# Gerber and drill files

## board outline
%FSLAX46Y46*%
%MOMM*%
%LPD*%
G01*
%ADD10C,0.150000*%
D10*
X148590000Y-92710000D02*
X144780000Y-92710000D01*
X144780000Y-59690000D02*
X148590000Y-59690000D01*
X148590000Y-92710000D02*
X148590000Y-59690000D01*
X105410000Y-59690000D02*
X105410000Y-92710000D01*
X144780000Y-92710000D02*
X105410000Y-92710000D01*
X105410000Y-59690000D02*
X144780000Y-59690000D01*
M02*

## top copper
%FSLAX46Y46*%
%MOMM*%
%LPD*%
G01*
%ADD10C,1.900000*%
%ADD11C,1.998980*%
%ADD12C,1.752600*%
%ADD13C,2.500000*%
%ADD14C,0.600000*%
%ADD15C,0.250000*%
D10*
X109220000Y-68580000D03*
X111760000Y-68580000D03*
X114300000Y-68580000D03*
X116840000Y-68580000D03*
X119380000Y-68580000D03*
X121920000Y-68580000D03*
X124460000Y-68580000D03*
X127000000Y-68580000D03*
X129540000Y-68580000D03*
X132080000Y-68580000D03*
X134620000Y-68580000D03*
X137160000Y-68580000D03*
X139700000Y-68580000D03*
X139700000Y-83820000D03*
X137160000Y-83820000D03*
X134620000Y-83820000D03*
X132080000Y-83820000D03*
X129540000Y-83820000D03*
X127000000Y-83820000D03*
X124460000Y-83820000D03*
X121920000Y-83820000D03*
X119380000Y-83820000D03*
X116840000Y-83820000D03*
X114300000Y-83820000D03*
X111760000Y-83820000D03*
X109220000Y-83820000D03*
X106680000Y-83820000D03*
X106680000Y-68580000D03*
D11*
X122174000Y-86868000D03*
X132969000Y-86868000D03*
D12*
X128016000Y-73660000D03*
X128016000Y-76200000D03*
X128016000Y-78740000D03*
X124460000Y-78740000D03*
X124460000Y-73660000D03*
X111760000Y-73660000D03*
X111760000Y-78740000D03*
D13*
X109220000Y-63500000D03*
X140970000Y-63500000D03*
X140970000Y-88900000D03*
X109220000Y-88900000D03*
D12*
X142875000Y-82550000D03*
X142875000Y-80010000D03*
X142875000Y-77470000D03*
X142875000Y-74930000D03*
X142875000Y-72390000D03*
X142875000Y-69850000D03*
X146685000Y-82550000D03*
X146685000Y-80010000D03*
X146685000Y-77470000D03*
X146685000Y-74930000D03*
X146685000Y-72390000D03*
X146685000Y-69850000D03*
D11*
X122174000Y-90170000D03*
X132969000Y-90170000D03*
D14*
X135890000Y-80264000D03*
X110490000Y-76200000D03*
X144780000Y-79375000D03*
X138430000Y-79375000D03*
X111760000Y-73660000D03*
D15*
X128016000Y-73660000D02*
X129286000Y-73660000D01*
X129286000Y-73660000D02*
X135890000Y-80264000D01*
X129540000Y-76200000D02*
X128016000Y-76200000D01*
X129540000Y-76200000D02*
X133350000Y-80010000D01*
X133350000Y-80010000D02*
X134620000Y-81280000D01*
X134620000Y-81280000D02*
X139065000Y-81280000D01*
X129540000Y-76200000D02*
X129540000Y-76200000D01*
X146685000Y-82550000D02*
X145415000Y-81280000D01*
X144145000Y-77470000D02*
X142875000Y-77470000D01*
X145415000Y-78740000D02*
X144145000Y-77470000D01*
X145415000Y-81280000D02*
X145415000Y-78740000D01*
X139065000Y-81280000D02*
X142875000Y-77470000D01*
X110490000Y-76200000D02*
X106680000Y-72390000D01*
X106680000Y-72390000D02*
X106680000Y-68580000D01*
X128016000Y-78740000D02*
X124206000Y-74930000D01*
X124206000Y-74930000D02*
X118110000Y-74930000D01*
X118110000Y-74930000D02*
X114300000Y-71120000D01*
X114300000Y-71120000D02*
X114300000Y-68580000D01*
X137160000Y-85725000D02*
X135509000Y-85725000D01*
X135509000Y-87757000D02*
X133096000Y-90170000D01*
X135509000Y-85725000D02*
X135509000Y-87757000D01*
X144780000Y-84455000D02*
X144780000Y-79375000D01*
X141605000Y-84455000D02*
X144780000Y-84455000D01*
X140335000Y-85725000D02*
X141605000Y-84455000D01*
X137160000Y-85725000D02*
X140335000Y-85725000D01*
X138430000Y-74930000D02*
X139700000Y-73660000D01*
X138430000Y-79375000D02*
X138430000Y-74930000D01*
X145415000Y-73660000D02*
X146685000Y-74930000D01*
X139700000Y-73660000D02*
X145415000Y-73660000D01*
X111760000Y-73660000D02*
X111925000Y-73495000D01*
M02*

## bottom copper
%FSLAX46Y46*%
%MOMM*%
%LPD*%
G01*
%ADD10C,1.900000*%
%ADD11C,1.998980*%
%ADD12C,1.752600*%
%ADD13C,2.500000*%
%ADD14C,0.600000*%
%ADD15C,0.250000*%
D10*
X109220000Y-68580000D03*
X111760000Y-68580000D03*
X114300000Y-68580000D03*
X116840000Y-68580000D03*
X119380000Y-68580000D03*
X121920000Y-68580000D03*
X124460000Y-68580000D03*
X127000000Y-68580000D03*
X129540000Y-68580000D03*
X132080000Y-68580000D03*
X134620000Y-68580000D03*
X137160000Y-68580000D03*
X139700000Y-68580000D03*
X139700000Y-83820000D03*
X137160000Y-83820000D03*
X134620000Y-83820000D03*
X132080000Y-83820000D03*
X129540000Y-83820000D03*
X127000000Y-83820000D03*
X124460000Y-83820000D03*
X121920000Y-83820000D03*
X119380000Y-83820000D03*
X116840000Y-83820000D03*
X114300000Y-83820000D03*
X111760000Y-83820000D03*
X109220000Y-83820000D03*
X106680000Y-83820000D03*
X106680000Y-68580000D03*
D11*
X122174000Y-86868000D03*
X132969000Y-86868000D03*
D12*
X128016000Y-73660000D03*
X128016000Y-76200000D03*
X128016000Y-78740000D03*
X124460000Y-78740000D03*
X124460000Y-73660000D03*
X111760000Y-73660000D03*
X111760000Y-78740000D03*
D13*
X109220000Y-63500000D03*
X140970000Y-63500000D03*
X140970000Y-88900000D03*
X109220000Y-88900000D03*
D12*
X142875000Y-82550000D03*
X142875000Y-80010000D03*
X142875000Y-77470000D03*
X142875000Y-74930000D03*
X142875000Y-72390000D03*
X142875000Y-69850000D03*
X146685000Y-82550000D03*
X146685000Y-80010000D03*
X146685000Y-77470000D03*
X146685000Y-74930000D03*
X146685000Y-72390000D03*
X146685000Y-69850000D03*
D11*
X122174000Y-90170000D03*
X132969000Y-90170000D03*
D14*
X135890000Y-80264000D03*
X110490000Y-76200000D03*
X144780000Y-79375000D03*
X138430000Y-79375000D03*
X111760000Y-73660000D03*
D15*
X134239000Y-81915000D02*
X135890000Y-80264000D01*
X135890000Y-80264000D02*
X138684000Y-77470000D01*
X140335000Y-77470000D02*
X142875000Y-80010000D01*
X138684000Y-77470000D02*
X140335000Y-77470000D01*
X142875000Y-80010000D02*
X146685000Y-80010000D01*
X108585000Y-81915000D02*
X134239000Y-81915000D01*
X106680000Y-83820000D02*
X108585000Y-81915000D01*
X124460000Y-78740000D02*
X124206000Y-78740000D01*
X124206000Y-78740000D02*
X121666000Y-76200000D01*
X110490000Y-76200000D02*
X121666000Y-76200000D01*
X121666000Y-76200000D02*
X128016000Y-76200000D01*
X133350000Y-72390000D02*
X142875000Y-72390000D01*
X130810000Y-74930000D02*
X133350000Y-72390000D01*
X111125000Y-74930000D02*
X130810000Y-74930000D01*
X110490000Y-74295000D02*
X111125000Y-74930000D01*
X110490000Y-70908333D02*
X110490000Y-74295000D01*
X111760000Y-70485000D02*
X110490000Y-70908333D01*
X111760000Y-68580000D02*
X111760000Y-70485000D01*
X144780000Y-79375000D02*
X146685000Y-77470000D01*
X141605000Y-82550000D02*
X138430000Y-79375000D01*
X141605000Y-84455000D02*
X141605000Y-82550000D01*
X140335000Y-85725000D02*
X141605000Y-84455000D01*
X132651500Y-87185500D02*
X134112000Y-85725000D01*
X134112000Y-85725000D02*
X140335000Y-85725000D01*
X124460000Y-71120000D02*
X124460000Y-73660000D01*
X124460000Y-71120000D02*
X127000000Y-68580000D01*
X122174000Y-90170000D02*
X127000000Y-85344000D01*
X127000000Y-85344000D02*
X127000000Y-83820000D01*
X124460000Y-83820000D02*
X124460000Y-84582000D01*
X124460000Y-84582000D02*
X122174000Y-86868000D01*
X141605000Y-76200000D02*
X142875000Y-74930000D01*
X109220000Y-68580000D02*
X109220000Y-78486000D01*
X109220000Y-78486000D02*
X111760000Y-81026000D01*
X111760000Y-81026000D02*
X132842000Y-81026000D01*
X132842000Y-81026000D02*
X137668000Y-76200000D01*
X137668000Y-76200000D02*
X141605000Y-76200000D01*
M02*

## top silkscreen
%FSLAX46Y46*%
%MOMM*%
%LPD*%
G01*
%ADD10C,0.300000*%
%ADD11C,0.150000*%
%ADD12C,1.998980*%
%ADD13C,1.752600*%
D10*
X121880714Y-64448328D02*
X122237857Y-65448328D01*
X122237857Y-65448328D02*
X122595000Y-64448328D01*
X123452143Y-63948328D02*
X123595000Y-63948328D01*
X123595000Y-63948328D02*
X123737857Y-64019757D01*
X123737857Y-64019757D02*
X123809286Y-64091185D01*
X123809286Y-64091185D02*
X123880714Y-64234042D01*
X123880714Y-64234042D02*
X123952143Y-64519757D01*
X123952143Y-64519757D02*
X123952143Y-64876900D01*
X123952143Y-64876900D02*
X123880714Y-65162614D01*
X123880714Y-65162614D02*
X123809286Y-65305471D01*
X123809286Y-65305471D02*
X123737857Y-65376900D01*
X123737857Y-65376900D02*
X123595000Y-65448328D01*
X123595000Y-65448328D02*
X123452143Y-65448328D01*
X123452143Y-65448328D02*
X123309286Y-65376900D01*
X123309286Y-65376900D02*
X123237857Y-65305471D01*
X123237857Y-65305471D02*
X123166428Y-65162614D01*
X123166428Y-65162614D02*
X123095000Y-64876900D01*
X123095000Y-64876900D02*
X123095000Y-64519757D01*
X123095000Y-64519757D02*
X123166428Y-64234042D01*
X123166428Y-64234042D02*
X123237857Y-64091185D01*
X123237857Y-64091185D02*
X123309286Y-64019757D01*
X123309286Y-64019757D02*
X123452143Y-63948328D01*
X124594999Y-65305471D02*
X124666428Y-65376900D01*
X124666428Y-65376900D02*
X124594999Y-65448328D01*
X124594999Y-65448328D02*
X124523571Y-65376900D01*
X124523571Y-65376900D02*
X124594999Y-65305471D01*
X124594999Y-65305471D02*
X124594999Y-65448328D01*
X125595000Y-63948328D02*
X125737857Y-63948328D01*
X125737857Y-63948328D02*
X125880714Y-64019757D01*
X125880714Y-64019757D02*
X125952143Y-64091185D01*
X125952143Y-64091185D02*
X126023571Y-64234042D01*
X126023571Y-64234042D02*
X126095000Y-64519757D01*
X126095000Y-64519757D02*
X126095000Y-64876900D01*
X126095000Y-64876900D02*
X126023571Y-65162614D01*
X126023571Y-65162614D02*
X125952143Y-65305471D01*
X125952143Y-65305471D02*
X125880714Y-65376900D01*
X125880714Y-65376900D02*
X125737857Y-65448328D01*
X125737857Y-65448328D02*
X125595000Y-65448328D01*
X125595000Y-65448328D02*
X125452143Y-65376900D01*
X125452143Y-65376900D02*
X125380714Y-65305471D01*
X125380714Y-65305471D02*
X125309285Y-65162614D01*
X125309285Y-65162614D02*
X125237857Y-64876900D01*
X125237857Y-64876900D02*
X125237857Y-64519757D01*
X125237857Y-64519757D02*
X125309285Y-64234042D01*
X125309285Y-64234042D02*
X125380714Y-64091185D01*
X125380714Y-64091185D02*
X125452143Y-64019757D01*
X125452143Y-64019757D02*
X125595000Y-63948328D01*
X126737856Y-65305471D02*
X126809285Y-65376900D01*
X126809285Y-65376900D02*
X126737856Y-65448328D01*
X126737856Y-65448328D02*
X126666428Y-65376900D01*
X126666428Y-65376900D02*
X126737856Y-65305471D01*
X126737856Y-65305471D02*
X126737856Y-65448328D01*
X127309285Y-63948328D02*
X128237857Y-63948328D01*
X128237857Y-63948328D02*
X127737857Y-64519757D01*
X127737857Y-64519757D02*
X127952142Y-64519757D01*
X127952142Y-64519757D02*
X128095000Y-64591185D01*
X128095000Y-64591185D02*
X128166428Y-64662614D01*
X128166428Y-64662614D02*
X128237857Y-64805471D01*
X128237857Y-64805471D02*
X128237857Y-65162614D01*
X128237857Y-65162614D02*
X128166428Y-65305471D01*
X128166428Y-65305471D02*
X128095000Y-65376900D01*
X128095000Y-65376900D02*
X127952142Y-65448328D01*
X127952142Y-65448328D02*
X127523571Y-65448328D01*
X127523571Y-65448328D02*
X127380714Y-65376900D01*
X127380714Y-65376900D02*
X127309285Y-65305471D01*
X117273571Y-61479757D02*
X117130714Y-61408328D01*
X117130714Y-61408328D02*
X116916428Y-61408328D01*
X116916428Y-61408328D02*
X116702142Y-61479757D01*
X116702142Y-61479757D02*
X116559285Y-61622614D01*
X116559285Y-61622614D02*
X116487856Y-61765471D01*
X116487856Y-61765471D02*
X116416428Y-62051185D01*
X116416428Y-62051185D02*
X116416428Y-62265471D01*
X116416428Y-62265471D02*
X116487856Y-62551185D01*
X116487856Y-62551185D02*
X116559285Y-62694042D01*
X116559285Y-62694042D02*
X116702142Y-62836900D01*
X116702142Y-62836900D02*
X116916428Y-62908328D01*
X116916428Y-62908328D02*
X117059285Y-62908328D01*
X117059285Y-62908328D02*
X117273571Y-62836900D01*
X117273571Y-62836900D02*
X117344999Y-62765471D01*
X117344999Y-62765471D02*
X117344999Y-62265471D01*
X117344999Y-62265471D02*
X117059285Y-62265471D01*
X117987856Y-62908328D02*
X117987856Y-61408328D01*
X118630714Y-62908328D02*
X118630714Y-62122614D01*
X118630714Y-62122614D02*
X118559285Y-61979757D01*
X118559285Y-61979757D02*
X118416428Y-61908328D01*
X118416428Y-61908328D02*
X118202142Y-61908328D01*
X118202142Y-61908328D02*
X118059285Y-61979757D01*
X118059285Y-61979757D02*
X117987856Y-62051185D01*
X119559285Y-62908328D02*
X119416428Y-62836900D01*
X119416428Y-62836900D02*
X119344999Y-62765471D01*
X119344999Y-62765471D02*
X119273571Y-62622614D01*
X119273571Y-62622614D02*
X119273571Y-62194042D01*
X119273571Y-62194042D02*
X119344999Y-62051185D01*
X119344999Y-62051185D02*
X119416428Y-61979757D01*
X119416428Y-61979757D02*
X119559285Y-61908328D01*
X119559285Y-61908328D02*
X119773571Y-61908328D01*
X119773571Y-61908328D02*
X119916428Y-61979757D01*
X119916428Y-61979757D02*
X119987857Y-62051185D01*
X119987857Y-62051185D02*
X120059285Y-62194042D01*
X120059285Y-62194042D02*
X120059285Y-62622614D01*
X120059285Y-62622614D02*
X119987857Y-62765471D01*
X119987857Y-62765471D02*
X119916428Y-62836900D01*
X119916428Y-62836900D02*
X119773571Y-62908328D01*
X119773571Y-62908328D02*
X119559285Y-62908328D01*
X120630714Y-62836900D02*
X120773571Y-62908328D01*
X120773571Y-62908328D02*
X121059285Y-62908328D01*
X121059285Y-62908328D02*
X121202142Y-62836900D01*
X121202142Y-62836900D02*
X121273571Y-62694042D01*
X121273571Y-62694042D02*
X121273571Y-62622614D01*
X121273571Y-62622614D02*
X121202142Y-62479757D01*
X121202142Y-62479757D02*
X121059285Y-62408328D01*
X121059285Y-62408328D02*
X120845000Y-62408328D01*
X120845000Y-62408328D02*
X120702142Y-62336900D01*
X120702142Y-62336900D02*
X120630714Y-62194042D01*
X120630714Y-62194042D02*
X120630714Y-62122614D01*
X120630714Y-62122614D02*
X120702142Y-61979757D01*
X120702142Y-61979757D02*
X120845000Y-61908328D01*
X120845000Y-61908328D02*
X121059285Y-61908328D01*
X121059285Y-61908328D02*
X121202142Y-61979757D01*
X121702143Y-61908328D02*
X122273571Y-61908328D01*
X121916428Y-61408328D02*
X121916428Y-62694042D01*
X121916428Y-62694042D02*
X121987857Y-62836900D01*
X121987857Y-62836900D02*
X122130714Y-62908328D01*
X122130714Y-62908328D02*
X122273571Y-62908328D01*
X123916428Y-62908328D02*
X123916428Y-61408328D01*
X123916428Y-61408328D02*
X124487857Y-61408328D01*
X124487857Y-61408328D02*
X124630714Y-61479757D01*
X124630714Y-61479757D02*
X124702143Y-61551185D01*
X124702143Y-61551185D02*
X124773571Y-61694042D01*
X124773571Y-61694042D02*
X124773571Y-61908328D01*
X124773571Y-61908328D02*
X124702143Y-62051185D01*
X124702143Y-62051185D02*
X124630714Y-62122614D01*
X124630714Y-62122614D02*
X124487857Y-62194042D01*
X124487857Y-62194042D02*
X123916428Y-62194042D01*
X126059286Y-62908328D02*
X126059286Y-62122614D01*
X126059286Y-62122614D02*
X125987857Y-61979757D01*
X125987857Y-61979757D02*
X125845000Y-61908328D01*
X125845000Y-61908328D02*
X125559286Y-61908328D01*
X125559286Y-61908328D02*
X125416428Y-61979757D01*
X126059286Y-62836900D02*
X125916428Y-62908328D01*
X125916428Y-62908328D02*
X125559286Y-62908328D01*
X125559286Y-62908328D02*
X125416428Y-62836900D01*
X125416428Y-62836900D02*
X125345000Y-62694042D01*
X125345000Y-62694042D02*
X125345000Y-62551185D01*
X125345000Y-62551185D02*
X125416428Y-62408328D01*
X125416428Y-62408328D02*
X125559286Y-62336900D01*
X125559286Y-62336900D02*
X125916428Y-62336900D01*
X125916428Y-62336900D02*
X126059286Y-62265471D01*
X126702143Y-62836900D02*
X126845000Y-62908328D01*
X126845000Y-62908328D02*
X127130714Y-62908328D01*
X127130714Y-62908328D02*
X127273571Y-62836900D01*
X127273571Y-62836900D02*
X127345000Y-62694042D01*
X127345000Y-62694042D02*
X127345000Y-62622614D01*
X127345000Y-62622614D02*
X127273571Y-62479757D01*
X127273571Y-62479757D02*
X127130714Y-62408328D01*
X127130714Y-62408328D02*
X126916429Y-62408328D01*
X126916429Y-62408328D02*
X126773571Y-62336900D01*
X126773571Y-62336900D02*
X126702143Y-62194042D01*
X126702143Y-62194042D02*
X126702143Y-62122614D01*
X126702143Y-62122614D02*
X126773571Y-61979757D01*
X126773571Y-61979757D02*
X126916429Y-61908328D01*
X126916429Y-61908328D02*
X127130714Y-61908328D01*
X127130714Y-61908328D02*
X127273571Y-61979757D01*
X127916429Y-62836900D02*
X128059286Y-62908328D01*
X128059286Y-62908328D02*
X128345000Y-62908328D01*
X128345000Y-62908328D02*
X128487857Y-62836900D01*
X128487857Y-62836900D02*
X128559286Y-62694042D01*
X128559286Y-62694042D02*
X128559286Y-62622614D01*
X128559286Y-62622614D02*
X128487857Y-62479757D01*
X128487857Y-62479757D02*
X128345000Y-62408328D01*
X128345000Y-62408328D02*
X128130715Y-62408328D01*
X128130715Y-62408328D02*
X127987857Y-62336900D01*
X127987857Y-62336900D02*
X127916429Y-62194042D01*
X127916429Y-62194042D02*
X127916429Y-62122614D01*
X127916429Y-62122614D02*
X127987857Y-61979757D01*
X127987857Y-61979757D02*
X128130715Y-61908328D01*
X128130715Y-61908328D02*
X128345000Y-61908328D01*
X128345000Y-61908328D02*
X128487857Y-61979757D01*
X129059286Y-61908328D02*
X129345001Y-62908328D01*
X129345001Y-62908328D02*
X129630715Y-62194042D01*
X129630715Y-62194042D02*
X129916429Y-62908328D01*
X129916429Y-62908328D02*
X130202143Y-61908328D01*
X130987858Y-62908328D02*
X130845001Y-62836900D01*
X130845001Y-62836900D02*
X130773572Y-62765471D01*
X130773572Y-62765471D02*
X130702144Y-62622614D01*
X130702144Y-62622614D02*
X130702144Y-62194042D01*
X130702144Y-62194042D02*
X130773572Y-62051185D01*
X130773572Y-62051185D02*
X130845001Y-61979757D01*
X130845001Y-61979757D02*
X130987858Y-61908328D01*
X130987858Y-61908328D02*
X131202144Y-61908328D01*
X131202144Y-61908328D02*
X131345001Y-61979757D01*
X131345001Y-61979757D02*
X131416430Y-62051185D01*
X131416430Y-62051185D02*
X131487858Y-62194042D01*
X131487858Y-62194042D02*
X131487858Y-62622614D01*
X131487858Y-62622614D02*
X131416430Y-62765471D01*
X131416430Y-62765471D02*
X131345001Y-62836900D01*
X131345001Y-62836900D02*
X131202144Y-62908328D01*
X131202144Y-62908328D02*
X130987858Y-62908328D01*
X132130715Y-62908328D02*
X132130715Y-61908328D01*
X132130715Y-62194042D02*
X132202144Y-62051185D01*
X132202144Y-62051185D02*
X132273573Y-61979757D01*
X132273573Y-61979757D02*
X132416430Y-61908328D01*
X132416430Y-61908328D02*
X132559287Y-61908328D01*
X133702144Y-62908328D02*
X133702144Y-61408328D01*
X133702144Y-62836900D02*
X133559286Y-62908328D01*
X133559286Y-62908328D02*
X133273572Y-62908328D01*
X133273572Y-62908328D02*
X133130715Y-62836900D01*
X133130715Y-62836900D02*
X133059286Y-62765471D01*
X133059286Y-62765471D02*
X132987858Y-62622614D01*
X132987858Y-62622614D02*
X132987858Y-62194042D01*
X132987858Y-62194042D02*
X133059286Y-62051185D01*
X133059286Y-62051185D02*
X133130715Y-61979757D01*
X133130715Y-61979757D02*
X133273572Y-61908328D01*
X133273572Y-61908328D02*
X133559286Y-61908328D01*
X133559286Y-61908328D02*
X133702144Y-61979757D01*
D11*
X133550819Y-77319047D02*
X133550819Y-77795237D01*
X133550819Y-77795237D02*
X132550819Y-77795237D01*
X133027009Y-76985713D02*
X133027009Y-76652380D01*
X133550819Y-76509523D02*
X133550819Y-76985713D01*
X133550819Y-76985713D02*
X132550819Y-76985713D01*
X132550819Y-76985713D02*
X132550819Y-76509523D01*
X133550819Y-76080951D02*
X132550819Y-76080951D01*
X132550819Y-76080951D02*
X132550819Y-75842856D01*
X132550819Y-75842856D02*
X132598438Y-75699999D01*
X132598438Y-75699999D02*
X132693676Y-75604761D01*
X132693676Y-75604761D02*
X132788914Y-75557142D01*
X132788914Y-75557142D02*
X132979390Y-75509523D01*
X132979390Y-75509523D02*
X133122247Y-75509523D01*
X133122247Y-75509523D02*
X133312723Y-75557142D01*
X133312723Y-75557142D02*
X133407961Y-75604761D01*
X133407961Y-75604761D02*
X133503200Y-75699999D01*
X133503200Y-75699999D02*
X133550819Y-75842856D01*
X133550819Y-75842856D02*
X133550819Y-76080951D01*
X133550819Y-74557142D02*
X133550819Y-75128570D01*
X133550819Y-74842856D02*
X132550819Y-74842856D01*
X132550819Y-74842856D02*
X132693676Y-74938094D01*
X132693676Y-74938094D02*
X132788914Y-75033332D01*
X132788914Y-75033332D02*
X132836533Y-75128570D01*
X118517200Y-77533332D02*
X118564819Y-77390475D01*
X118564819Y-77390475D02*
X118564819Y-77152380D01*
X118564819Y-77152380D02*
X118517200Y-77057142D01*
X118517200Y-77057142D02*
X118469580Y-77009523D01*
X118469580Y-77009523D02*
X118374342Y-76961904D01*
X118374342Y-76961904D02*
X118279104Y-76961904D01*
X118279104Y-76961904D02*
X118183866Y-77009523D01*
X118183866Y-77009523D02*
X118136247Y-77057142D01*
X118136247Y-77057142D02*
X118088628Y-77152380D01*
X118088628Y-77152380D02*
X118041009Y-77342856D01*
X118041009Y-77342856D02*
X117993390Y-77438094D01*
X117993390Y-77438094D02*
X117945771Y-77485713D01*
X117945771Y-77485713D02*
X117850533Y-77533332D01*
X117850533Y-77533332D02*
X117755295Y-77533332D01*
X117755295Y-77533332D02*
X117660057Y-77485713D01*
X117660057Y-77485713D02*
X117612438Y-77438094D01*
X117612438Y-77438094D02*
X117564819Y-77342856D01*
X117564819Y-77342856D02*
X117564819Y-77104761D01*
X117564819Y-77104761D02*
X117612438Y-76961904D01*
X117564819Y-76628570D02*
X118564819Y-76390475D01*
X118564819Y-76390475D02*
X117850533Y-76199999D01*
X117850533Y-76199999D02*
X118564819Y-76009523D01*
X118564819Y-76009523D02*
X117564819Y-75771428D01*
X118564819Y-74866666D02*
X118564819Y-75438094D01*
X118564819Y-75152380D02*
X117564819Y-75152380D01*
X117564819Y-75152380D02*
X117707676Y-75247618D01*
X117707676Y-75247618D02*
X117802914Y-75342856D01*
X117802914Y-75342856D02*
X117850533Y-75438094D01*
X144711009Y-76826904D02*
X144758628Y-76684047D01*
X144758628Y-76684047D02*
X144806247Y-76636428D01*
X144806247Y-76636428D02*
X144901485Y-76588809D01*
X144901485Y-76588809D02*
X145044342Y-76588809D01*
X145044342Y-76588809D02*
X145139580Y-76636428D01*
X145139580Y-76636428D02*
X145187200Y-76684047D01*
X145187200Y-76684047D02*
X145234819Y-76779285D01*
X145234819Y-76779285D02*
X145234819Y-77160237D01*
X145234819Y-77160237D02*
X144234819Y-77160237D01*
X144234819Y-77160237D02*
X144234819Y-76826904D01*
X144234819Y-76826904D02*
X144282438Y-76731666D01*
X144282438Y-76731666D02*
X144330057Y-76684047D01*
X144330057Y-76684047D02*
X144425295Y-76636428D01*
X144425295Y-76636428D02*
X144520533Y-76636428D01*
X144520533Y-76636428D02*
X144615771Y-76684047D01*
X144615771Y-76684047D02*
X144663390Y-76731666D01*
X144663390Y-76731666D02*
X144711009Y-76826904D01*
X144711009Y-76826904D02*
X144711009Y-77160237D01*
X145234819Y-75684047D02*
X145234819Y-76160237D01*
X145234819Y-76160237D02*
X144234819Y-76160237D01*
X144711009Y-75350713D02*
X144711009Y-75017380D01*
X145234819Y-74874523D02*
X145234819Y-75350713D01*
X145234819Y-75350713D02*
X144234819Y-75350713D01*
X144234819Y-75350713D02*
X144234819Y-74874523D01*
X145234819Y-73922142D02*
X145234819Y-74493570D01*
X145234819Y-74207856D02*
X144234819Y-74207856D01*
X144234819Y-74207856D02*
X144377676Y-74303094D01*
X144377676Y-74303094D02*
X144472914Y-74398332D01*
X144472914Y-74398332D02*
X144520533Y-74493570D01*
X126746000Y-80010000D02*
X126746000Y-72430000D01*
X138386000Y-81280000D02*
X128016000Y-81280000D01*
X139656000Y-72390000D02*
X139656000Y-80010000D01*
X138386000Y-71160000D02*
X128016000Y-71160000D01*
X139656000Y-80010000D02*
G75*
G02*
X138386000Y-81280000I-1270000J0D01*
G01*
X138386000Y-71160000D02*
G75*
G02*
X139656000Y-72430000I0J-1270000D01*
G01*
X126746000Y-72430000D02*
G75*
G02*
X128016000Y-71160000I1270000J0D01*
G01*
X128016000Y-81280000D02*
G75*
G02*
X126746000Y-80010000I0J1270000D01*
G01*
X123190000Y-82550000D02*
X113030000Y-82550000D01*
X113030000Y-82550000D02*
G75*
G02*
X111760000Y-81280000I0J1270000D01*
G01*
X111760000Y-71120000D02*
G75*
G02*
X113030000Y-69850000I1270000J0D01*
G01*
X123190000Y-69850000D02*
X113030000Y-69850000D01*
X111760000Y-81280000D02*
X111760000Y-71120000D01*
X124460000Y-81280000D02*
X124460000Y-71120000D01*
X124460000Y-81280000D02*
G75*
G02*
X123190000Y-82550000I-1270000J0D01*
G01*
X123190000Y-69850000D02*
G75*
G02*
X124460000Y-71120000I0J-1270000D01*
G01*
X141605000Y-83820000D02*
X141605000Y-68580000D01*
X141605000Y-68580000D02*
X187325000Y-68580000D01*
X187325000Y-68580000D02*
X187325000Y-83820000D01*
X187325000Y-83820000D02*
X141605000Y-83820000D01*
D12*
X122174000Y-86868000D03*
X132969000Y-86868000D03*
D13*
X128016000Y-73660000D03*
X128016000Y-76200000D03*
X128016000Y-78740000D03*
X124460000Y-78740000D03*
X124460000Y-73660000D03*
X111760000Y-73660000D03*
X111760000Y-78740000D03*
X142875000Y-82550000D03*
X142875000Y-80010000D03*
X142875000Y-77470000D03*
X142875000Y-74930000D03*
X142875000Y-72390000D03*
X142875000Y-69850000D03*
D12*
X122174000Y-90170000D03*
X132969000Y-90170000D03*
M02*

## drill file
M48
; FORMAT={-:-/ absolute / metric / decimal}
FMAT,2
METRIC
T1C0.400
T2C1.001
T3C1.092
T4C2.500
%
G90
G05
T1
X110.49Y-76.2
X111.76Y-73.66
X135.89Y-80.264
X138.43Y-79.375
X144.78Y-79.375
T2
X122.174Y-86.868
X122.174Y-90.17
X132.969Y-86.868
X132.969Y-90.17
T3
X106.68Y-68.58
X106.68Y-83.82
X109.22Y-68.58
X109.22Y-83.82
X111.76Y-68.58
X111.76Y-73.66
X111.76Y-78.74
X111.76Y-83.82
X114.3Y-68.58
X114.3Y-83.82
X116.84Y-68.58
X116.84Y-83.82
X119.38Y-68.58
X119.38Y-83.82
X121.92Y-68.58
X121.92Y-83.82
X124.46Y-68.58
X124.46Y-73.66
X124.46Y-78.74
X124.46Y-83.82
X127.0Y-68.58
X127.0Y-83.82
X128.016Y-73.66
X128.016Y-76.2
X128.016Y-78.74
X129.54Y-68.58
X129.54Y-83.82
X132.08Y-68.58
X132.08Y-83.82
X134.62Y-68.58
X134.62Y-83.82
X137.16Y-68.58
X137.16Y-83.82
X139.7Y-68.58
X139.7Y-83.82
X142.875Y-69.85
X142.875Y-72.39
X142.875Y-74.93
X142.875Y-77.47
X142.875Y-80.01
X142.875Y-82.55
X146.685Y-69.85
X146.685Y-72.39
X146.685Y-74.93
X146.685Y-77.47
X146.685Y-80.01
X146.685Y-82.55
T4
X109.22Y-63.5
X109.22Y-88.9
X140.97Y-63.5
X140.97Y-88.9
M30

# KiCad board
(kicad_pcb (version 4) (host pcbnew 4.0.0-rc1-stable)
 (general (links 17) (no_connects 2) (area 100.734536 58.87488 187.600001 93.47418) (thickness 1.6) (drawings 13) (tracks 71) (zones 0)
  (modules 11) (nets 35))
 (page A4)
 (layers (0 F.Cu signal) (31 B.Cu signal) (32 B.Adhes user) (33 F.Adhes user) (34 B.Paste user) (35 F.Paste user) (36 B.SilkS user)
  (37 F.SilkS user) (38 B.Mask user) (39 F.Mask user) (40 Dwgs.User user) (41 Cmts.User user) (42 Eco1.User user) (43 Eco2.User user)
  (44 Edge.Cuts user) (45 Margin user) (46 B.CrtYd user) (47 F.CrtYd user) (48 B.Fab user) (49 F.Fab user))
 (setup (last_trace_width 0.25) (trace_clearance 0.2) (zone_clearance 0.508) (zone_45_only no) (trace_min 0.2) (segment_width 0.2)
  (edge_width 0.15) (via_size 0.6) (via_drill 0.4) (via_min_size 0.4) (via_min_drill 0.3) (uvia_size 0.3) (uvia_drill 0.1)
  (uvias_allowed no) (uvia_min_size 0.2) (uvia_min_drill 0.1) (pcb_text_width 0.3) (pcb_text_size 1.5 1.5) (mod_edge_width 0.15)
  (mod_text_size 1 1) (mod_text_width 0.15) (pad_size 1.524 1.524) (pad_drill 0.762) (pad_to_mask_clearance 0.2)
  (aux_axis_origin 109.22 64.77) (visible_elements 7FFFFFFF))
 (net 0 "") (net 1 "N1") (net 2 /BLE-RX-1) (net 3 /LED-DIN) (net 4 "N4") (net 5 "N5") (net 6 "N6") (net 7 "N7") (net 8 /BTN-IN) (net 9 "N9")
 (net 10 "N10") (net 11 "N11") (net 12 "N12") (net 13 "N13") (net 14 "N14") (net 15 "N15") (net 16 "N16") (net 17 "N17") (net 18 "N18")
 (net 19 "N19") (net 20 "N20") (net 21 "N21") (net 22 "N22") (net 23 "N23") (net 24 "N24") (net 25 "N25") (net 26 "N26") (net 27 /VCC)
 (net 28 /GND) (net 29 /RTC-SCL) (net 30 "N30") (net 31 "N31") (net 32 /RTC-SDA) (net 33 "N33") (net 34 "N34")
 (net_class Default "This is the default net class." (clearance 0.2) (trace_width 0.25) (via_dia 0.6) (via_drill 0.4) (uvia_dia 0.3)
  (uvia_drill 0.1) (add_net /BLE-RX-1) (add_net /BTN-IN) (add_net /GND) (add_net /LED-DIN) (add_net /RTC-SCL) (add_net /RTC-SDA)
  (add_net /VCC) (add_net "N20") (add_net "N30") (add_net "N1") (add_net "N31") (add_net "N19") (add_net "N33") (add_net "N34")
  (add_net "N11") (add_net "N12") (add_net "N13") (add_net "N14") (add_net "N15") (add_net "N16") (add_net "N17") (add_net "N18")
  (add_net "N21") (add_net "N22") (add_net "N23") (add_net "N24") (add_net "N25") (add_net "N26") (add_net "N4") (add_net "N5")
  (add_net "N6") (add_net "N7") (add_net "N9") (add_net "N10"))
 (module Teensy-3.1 (layer B.Cu) (at 109.22 68.58)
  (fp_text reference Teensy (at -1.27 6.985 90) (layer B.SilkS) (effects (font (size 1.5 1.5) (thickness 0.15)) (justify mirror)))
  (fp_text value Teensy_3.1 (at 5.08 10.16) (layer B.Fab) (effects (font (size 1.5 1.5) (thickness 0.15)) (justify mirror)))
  (pad 0 thru_hole circle (at 0 0) (size 1.9 1.9) (drill 1.0922) (layers *.Cu *.Mask B.SilkS) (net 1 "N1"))
  (pad 1 thru_hole circle (at 2.54 0) (size 1.9 1.9) (drill 1.0922) (layers *.Cu *.Mask B.SilkS) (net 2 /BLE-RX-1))
  (pad 2 thru_hole circle (at 5.08 0) (size 1.9 1.9) (drill 1.0922) (layers *.Cu *.Mask B.SilkS) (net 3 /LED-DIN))
  (pad 3 thru_hole circle (at 7.62 0) (size 1.9 1.9) (drill 1.0922) (layers *.Cu *.Mask B.SilkS) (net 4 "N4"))
  (pad 4 thru_hole circle (at 10.16 0) (size 1.9 1.9) (drill 1.0922) (layers *.Cu *.Mask B.SilkS) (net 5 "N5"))
  (pad 5 thru_hole circle (at 12.7 0) (size 1.9 1.9) (drill 1.0922) (layers *.Cu *.Mask B.SilkS) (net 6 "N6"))
  (pad 6 thru_hole circle (at 15.24 0) (size 1.9 1.9) (drill 1.0922) (layers *.Cu *.Mask B.SilkS) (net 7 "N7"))
  (pad 7 thru_hole circle (at 17.78 0) (size 1.9 1.9) (drill 1.0922) (layers *.Cu *.Mask B.SilkS) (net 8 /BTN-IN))
  (pad 8 thru_hole circle (at 20.32 0) (size 1.9 1.9) (drill 1.0922) (layers *.Cu *.Mask B.SilkS) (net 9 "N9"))
  (pad 9 thru_hole circle (at 22.86 0) (size 1.9 1.9) (drill 1.0922) (layers *.Cu *.Mask B.SilkS) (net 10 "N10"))
  (pad 10 thru_hole circle (at 25.4 0) (size 1.9 1.9) (drill 1.0922) (layers *.Cu *.Mask B.SilkS) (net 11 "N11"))
  (pad 11 thru_hole circle (at 27.94 0) (size 1.9 1.9) (drill 1.0922) (layers *.Cu *.Mask B.SilkS) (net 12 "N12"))
  (pad 12 thru_hole circle (at 30.48 0) (size 1.9 1.9) (drill 1.0922) (layers *.Cu *.Mask B.SilkS) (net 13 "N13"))
  (pad 13 thru_hole circle (at 30.48 15.24) (size 1.9 1.9) (drill 1.0922) (layers *.Cu *.Mask B.SilkS) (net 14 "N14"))
  (pad 14 thru_hole circle (at 27.94 15.24) (size 1.9 1.9) (drill 1.0922) (layers *.Cu *.Mask B.SilkS) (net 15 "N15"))
  (pad 15 thru_hole circle (at 25.4 15.24) (size 1.9 1.9) (drill 1.0922) (layers *.Cu *.Mask B.SilkS) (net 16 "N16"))
  (pad 16 thru_hole circle (at 22.86 15.24) (size 1.9 1.9) (drill 1.0922) (layers *.Cu *.Mask B.SilkS) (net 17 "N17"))
  (pad 17 thru_hole circle (at 20.32 15.24) (size 1.9 1.9) (drill 1.0922) (layers *.Cu *.Mask B.SilkS) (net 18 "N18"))
  (pad 18 thru_hole circle (at 17.78 15.24) (size 1.9 1.9) (drill 1.0922) (layers *.Cu *.Mask B.SilkS) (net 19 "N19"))
  (pad 19 thru_hole circle (at 15.24 15.24) (size 1.9 1.9) (drill 1.0922) (layers *.Cu *.Mask B.SilkS) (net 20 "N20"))
  (pad 20 thru_hole circle (at 12.7 15.24) (size 1.9 1.9) (drill 1.0922) (layers *.Cu *.Mask B.SilkS) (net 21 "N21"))
  (pad 21 thru_hole circle (at 10.16 15.24) (size 1.9 1.9) (drill 1.0922) (layers *.Cu *.Mask B.SilkS) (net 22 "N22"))
  (pad 22 thru_hole circle (at 7.62 15.24) (size 1.9 1.9) (drill 1.0922) (layers *.Cu *.Mask B.SilkS) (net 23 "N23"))
  (pad 23 thru_hole circle (at 5.08 15.24) (size 1.9 1.9) (drill 1.0922) (layers *.Cu *.Mask B.SilkS) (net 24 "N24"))
  (pad 24 thru_hole circle (at 2.54 15.24) (size 1.9 1.9) (drill 1.0922) (layers *.Cu *.Mask B.SilkS) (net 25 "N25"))
  (pad 25 thru_hole circle (at 0 15.24) (size 1.9 1.9) (drill 1.0922) (layers *.Cu *.Mask B.SilkS) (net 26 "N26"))
  (pad 26 thru_hole circle (at -2.54 15.24) (size 1.9 1.9) (drill 1.0922) (layers *.Cu *.Mask B.SilkS) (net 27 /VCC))
  (pad 27 thru_hole circle (at -2.54 0) (size 1.9 1.9) (drill 1.0922) (layers *.Cu *.Mask B.SilkS) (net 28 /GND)))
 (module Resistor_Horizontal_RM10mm (layer B.Cu) (at 127.254 86.868)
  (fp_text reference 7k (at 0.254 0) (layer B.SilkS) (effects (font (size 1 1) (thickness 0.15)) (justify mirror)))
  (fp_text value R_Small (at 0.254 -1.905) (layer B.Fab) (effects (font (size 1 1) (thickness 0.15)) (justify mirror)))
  (pad 1 thru_hole circle (at -5.08 0) (size 1.99898 1.99898) (drill 1.00076) (layers *.Cu *.SilkS *.Mask) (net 20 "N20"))
  (pad 2 thru_hole circle (at 5.715 0) (size 1.99898 1.99898) (drill 1.00076) (layers *.Cu *.SilkS *.Mask) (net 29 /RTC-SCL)))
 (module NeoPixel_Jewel (layer F.Cu) (at 126.746 81.28 90)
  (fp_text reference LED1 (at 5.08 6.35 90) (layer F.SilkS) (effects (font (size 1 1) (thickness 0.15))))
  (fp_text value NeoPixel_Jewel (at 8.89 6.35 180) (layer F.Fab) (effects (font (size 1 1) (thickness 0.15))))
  (fp_line (start 1.27 0) (end 8.85 0) (layer F.SilkS) (width 0.15))
  (fp_line (start 0 11.64) (end 0 1.27) (layer F.SilkS) (width 0.15))
  (fp_line (start 8.89 12.91) (end 1.27 12.91) (layer F.SilkS) (width 0.15))
  (fp_line (start 10.12 11.64) (end 10.12 1.27) (layer F.SilkS) (width 0.15))
  (fp_arc (start 1.27 11.64) (end 1.27 12.91) (angle 90) (layer F.SilkS) (width 0.15))
  (fp_arc (start 8.85 11.64) (end 10.12 11.64) (angle 90) (layer F.SilkS) (width 0.15))
  (fp_arc (start 8.85 1.27) (end 8.85 0) (angle 90) (layer F.SilkS) (width 0.15))
  (fp_arc (start 1.27 1.27) (end 0 1.27) (angle 90) (layer F.SilkS) (width 0.15))
  (pad 1 thru_hole circle (at 7.62 1.27 90) (size 1.7526 1.7526) (drill 1.0922) (layers *.Cu *.Mask F.SilkS) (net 27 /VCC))
  (pad 2 thru_hole circle (at 5.08 1.27 90) (size 1.7526 1.7526) (drill 1.0922) (layers *.Cu *.Mask F.SilkS) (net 28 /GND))
  (pad 3 thru_hole circle (at 2.54 1.27 90) (size 1.7526 1.7526) (drill 1.0922) (layers *.Cu *.Mask F.SilkS) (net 3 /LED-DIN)))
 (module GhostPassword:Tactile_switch (layer F.Cu) (at 118.11 76.2 270)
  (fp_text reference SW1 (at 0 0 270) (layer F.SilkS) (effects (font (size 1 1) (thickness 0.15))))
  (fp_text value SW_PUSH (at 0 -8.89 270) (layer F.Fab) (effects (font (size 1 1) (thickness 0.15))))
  (fp_line (start 6.35 -5.08) (end 6.35 5.08) (layer F.SilkS) (width 0.15))
  (fp_arc (start 5.08 5.08) (end 6.35 5.08) (angle 90) (layer F.SilkS) (width 0.15))
  (fp_arc (start -5.08 5.08) (end -5.08 6.35) (angle 90) (layer F.SilkS) (width 0.15))
  (fp_line (start -6.35 -5.08) (end -6.35 5.08) (layer F.SilkS) (width 0.15))
  (fp_line (start 5.08 6.35) (end -5.08 6.35) (layer F.SilkS) (width 0.15))
  (fp_line (start 5.08 -6.35) (end -5.08 -6.35) (layer F.SilkS) (width 0.15))
  (fp_arc (start 5.08 -5.08) (end 5.08 -6.35) (angle 90) (layer F.SilkS) (width 0.15))
  (fp_arc (start -5.08 -5.08) (end -6.35 -5.08) (angle 90) (layer F.SilkS) (width 0.15))
  (pad 2 thru_hole circle (at 2.54 -6.35 270) (size 1.7526 1.7526) (drill 1.0922) (layers *.Cu *.Mask F.SilkS) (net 28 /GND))
  (pad 1 thru_hole circle (at -2.54 -6.35 270) (size 1.7526 1.7526) (drill 1.0922) (layers *.Cu *.Mask F.SilkS) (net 8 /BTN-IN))
  (pad 1 thru_hole circle (at -2.54 6.35 270) (size 1.7526 1.7526) (drill 1.0922) (layers *.Cu *.Mask F.SilkS) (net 8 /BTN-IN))
  (pad 2 thru_hole circle (at 2.54 6.35 270) (size 1.7526 1.7526) (drill 1.0922) (layers *.Cu *.Mask F.SilkS) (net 28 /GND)))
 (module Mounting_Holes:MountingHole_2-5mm (layer F.Cu) (at 109.22 63.5)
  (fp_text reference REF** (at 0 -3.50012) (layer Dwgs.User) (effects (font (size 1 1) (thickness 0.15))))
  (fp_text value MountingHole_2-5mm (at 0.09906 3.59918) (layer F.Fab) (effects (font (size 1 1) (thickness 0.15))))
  (pad 1 thru_hole circle (at 0 0) (size 2.5 2.5) (drill 2.5) (layers)))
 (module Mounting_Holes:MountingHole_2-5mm (layer F.Cu) (at 140.97 63.5)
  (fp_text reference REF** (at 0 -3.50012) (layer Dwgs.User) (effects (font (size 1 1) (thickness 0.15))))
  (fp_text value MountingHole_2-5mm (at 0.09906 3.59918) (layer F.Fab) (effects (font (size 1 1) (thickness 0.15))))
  (pad 1 thru_hole circle (at 0 0) (size 2.5 2.5) (drill 2.5) (layers)))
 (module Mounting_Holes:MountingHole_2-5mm (layer F.Cu) (at 140.97 88.9)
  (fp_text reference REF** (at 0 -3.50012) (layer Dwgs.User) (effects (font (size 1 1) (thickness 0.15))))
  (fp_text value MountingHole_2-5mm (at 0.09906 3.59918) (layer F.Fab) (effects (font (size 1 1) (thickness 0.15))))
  (pad 1 thru_hole circle (at 0 0) (size 2.5 2.5) (drill 2.5) (layers)))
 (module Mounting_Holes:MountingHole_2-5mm (layer F.Cu) (at 109.22 88.9)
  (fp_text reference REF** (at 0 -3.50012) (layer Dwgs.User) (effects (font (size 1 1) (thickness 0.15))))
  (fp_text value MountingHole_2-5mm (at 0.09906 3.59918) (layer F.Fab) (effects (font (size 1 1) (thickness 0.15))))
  (pad 1 thru_hole circle (at 0 0) (size 2.5 2.5) (drill 2.5) (layers)))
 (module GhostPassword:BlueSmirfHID (layer F.Cu) (at 141.605 83.82 90)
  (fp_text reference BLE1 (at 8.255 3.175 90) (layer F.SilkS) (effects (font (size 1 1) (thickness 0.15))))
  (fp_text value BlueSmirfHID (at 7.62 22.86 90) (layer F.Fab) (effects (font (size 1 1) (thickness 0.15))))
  (fp_line (start 0 0) (end 15.24 0) (layer F.SilkS) (width 0.15))
  (fp_line (start 15.24 0) (end 15.24 45.72) (layer F.SilkS) (width 0.15))
  (fp_line (start 15.24 45.72) (end 0 45.72) (layer F.SilkS) (width 0.15))
  (fp_line (start 0 45.72) (end 0 0) (layer F.SilkS) (width 0.15))
  (pad 1 thru_hole circle (at 1.27 1.27 90) (size 1.7526 1.7526) (drill 1.0922) (layers *.Cu *.Mask F.SilkS) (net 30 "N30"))
  (pad 2 thru_hole circle (at 3.81 1.27 90) (size 1.7526 1.7526) (drill 1.0922) (layers *.Cu *.Mask F.SilkS) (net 27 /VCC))
  (pad 3 thru_hole circle (at 6.35 1.27 90) (size 1.7526 1.7526) (drill 1.0922) (layers *.Cu *.Mask F.SilkS) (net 28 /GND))
  (pad 4 thru_hole circle (at 8.89 1.27 90) (size 1.7526 1.7526) (drill 1.0922) (layers *.Cu *.Mask F.SilkS) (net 1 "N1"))
  (pad 5 thru_hole circle (at 11.43 1.27 90) (size 1.7526 1.7526) (drill 1.0922) (layers *.Cu *.Mask F.SilkS) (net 2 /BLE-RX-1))
  (pad 6 thru_hole circle (at 13.97 1.27 90) (size 1.7526 1.7526) (drill 1.0922) (layers *.Cu *.Mask F.SilkS) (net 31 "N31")))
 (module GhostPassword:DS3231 (layer B.Cu) (at 144.145 64.77 270)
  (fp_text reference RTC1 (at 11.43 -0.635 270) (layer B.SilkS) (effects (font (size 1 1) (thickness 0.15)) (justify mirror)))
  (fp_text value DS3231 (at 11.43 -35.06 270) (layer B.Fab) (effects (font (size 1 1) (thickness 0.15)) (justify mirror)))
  (pad 1 thru_hole circle (at 17.78 -2.54 270) (size 1.7526 1.7526) (drill 1.0922) (layers *.Cu *.Mask B.SilkS) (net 28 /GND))
  (pad 2 thru_hole circle (at 15.24 -2.54 270) (size 1.7526 1.7526) (drill 1.0922) (layers *.Cu *.Mask B.SilkS) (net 27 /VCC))
  (pad 3 thru_hole circle (at 12.7 -2.54 270) (size 1.7526 1.7526) (drill 1.0922) (layers *.Cu *.Mask B.SilkS) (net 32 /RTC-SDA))
  (pad 4 thru_hole circle (at 10.16 -2.54 270) (size 1.7526 1.7526) (drill 1.0922) (layers *.Cu *.Mask B.SilkS) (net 29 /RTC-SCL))
  (pad 5 thru_hole circle (at 7.62 -2.54 270) (size 1.7526 1.7526) (drill 1.0922) (layers *.Cu *.Mask B.SilkS) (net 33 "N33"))
  (pad 6 thru_hole circle (at 5.08 -2.54 270) (size 1.7526 1.7526) (drill 1.0922) (layers *.Cu *.Mask B.SilkS) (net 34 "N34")))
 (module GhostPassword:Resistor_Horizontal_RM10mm (layer B.Cu) (at 127.254 90.17)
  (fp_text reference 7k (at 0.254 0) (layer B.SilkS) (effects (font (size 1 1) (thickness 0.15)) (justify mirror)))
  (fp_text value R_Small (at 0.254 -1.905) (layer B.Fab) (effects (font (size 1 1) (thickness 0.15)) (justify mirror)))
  (pad 1 thru_hole circle (at -5.08 0) (size 1.99898 1.99898) (drill 1.00076) (layers *.Cu *.SilkS *.Mask) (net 19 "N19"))
  (pad 2 thru_hole circle (at 5.715 0) (size 1.99898 1.99898) (drill 1.00076) (layers *.Cu *.SilkS *.Mask) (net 32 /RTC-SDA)))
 (gr_line (start 148.59 92.71) (end 144.78 92.71) (angle 90) (layer Edge.Cuts) (width 0.15))
 (gr_line (start 144.78 59.69) (end 148.59 59.69) (angle 90) (layer Edge.Cuts) (width 0.15))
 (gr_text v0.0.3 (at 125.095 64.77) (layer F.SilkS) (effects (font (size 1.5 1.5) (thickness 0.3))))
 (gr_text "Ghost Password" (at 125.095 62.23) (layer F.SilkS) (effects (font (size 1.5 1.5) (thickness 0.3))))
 (gr_line (start 148.59 92.71) (end 148.59 59.69) (angle 90) (layer Edge.Cuts) (width 0.15))
 (gr_line (start 105.41 59.69) (end 105.41 92.71) (angle 90) (layer Edge.Cuts) (width 0.15))
 (gr_line (start 144.78 92.71) (end 105.41 92.71) (angle 90) (layer Edge.Cuts) (width 0.15))
 (gr_line (start 105.41 59.69) (end 144.78 59.69) (angle 90) (layer Edge.Cuts) (width 0.15))
 (segment (start 128.016 73.66) (end 129.286 73.66) (width 0.25) (layer F.Cu) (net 27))
 (via (at 135.89 80.264) (size 0.6) (drill 0.4) (layers F.Cu B.Cu) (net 27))
 (segment (start 129.286 73.66) (end 135.89 80.264) (width 0.25) (layer F.Cu) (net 27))
 (segment (start 134.239 81.915) (end 135.89 80.264) (width 0.25) (layer B.Cu) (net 27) (status 20))
 (segment (start 135.89 80.264) (end 138.684 77.47) (width 0.25) (layer B.Cu) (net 27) (status 20))
 (segment (start 140.335 77.47) (end 142.875 80.01) (width 0.25) (layer B.Cu) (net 27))
 (segment (start 138.684 77.47) (end 140.335 77.47) (width 0.25) (layer B.Cu) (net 27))
 (segment (start 142.875 80.01) (end 146.685 80.01) (width 0.25) (layer B.Cu) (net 27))
 (segment (start 108.585 81.915) (end 134.239 81.915) (width 0.25) (layer B.Cu) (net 27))
 (segment (start 106.68 83.82) (end 108.585 81.915) (width 0.25) (layer B.Cu) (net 27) (status 10))
 (segment (start 129.54 76.2) (end 128.016 76.2) (width 0.25) (layer F.Cu) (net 28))
 (segment (start 124.46 78.74) (end 124.206 78.74) (width 0.25) (layer B.Cu) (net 28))
 (segment (start 124.206 78.74) (end 121.666 76.2) (width 0.25) (layer B.Cu) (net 28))
 (segment (start 110.49 76.2) (end 121.666 76.2) (width 0.25) (layer B.Cu) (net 28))
 (segment (start 121.666 76.2) (end 128.016 76.2) (width 0.25) (layer B.Cu) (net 28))
 (via (at 110.49 76.2) (size 0.6) (drill 0.4) (layers F.Cu B.Cu) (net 28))
 (segment (start 129.54 76.2) (end 133.35 80.01) (width 0.25) (layer F.Cu) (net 28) (status 10))
 (segment (start 133.35 80.01) (end 134.62 81.28) (width 0.25) (layer F.Cu) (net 28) (status 10))
 (segment (start 134.62 81.28) (end 139.065 81.28) (width 0.25) (layer F.Cu) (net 28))
 (segment (start 129.54 76.2) (end 129.54 76.2) (width 0.25) (layer F.Cu) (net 28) (status 10))
 (segment (start 146.685 82.55) (end 145.415 81.28) (width 0.25) (layer F.Cu) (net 28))
 (segment (start 144.145 77.47) (end 142.875 77.47) (width 0.25) (layer F.Cu) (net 28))
 (segment (start 145.415 78.74) (end 144.145 77.47) (width 0.25) (layer F.Cu) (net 28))
 (segment (start 145.415 81.28) (end 145.415 78.74) (width 0.25) (layer F.Cu) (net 28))
 (segment (start 139.065 81.28) (end 142.875 77.47) (width 0.25) (layer F.Cu) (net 28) (status 20))
 (segment (start 110.49 76.2) (end 106.68 72.39) (width 0.25) (layer F.Cu) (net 28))
 (segment (start 106.68 72.39) (end 106.68 68.58) (width 0.25) (layer F.Cu) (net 28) (status 20))
 (segment (start 133.35 72.39) (end 142.875 72.39) (width 0.25) (layer B.Cu) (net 2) (status 20))
 (segment (start 130.81 74.93) (end 133.35 72.39) (width 0.25) (layer B.Cu) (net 2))
 (segment (start 111.125 74.93) (end 130.81 74.93) (width 0.25) (layer B.Cu) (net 2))
 (segment (start 110.49 74.295) (end 111.125 74.93) (width 0.25) (layer B.Cu) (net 2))
 (segment (start 110.49 70.908333) (end 110.49 74.295) (width 0.25) (layer B.Cu) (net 2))
 (segment (start 111.76 70.485) (end 110.49 70.908333) (width 0.25) (layer B.Cu) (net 2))
 (segment (start 111.76 68.58) (end 111.76 70.485) (width 0.25) (layer B.Cu) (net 2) (status 10))
 (segment (start 128.016 78.74) (end 124.206 74.93) (width 0.25) (layer F.Cu) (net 3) (status 10))
 (segment (start 124.206 74.93) (end 118.11 74.93) (width 0.25) (layer F.Cu) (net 3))
 (segment (start 118.11 74.93) (end 114.3 71.12) (width 0.25) (layer F.Cu) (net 3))
 (segment (start 114.3 71.12) (end 114.3 68.58) (width 0.25) (layer F.Cu) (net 3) (status 20))
 (segment (start 137.16 85.725) (end 135.509 85.725) (width 0.25) (layer F.Cu) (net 32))
 (segment (start 135.509 87.757) (end 133.096 90.17) (width 0.25) (layer F.Cu) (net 32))
 (segment (start 135.509 85.725) (end 135.509 87.757) (width 0.25) (layer F.Cu) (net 32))
 (segment (start 144.78 79.375) (end 146.685 77.47) (width 0.25) (layer B.Cu) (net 32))
 (via (at 144.78 79.375) (size 0.6) (drill 0.4) (layers F.Cu B.Cu) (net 32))
 (segment (start 144.78 84.455) (end 144.78 79.375) (width 0.25) (layer F.Cu) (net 32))
 (segment (start 141.605 84.455) (end 144.78 84.455) (width 0.25) (layer F.Cu) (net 32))
 (segment (start 140.335 85.725) (end 141.605 84.455) (width 0.25) (layer F.Cu) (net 32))
 (segment (start 137.16 85.725) (end 140.335 85.725) (width 0.25) (layer F.Cu) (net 32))
 (segment (start 138.43 74.93) (end 139.7 73.66) (width 0.25) (layer F.Cu) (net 29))
 (segment (start 138.43 79.375) (end 138.43 74.93) (width 0.25) (layer F.Cu) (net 29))
 (via (at 138.43 79.375) (size 0.6) (drill 0.4) (layers F.Cu B.Cu) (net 29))
 (segment (start 141.605 82.55) (end 138.43 79.375) (width 0.25) (layer B.Cu) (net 29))
 (segment (start 141.605 84.455) (end 141.605 82.55) (width 0.25) (layer B.Cu) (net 29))
 (segment (start 140.335 85.725) (end 141.605 84.455) (width 0.25) (layer B.Cu) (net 29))
 (segment (start 132.6515 87.1855) (end 134.112 85.725) (width 0.25) (layer B.Cu) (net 29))
 (segment (start 145.415 73.66) (end 146.685 74.93) (width 0.25) (layer F.Cu) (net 29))
 (segment (start 139.7 73.66) (end 145.415 73.66) (width 0.25) (layer F.Cu) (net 29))
 (segment (start 134.112 85.725) (end 140.335 85.725) (width 0.25) (layer B.Cu) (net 29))
 (segment (start 111.76 73.66) (end 111.925 73.495) (width 0.25) (layer F.Cu) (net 8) (status 30))
 (via (at 111.76 73.66) (size 0.6) (drill 0.4) (layers F.Cu B.Cu) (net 8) (status 30))
 (segment (start 124.46 71.12) (end 124.46 73.66) (width 0.25) (layer B.Cu) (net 8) (status 20))
 (segment (start 124.46 71.12) (end 127 68.58) (width 0.25) (layer B.Cu) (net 8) (status 10))
 (segment (start 122.174 90.17) (end 127 85.344) (width 0.25) (layer B.Cu) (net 19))
 (segment (start 127 85.344) (end 127 83.82) (width 0.25) (layer B.Cu) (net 19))
 (segment (start 124.46 83.82) (end 124.46 84.582) (width 0.25) (layer B.Cu) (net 20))
 (segment (start 124.46 84.582) (end 122.174 86.868) (width 0.25) (layer B.Cu) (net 20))
 (segment (start 141.605 76.2) (end 142.875 74.93) (width 0.25) (layer B.Cu) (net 1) (status 20))
 (segment (start 109.22 68.58) (end 109.22 78.486) (width 0.25) (layer B.Cu) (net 1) (status 10))
 (segment (start 109.22 78.486) (end 111.76 81.026) (width 0.25) (layer B.Cu) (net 1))
 (segment (start 111.76 81.026) (end 132.842 81.026) (width 0.25) (layer B.Cu) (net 1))
 (segment (start 132.842 81.026) (end 137.668 76.2) (width 0.25) (layer B.Cu) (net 1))
 (segment (start 137.668 76.2) (end 141.605 76.2) (width 0.25) (layer B.Cu) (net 1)))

